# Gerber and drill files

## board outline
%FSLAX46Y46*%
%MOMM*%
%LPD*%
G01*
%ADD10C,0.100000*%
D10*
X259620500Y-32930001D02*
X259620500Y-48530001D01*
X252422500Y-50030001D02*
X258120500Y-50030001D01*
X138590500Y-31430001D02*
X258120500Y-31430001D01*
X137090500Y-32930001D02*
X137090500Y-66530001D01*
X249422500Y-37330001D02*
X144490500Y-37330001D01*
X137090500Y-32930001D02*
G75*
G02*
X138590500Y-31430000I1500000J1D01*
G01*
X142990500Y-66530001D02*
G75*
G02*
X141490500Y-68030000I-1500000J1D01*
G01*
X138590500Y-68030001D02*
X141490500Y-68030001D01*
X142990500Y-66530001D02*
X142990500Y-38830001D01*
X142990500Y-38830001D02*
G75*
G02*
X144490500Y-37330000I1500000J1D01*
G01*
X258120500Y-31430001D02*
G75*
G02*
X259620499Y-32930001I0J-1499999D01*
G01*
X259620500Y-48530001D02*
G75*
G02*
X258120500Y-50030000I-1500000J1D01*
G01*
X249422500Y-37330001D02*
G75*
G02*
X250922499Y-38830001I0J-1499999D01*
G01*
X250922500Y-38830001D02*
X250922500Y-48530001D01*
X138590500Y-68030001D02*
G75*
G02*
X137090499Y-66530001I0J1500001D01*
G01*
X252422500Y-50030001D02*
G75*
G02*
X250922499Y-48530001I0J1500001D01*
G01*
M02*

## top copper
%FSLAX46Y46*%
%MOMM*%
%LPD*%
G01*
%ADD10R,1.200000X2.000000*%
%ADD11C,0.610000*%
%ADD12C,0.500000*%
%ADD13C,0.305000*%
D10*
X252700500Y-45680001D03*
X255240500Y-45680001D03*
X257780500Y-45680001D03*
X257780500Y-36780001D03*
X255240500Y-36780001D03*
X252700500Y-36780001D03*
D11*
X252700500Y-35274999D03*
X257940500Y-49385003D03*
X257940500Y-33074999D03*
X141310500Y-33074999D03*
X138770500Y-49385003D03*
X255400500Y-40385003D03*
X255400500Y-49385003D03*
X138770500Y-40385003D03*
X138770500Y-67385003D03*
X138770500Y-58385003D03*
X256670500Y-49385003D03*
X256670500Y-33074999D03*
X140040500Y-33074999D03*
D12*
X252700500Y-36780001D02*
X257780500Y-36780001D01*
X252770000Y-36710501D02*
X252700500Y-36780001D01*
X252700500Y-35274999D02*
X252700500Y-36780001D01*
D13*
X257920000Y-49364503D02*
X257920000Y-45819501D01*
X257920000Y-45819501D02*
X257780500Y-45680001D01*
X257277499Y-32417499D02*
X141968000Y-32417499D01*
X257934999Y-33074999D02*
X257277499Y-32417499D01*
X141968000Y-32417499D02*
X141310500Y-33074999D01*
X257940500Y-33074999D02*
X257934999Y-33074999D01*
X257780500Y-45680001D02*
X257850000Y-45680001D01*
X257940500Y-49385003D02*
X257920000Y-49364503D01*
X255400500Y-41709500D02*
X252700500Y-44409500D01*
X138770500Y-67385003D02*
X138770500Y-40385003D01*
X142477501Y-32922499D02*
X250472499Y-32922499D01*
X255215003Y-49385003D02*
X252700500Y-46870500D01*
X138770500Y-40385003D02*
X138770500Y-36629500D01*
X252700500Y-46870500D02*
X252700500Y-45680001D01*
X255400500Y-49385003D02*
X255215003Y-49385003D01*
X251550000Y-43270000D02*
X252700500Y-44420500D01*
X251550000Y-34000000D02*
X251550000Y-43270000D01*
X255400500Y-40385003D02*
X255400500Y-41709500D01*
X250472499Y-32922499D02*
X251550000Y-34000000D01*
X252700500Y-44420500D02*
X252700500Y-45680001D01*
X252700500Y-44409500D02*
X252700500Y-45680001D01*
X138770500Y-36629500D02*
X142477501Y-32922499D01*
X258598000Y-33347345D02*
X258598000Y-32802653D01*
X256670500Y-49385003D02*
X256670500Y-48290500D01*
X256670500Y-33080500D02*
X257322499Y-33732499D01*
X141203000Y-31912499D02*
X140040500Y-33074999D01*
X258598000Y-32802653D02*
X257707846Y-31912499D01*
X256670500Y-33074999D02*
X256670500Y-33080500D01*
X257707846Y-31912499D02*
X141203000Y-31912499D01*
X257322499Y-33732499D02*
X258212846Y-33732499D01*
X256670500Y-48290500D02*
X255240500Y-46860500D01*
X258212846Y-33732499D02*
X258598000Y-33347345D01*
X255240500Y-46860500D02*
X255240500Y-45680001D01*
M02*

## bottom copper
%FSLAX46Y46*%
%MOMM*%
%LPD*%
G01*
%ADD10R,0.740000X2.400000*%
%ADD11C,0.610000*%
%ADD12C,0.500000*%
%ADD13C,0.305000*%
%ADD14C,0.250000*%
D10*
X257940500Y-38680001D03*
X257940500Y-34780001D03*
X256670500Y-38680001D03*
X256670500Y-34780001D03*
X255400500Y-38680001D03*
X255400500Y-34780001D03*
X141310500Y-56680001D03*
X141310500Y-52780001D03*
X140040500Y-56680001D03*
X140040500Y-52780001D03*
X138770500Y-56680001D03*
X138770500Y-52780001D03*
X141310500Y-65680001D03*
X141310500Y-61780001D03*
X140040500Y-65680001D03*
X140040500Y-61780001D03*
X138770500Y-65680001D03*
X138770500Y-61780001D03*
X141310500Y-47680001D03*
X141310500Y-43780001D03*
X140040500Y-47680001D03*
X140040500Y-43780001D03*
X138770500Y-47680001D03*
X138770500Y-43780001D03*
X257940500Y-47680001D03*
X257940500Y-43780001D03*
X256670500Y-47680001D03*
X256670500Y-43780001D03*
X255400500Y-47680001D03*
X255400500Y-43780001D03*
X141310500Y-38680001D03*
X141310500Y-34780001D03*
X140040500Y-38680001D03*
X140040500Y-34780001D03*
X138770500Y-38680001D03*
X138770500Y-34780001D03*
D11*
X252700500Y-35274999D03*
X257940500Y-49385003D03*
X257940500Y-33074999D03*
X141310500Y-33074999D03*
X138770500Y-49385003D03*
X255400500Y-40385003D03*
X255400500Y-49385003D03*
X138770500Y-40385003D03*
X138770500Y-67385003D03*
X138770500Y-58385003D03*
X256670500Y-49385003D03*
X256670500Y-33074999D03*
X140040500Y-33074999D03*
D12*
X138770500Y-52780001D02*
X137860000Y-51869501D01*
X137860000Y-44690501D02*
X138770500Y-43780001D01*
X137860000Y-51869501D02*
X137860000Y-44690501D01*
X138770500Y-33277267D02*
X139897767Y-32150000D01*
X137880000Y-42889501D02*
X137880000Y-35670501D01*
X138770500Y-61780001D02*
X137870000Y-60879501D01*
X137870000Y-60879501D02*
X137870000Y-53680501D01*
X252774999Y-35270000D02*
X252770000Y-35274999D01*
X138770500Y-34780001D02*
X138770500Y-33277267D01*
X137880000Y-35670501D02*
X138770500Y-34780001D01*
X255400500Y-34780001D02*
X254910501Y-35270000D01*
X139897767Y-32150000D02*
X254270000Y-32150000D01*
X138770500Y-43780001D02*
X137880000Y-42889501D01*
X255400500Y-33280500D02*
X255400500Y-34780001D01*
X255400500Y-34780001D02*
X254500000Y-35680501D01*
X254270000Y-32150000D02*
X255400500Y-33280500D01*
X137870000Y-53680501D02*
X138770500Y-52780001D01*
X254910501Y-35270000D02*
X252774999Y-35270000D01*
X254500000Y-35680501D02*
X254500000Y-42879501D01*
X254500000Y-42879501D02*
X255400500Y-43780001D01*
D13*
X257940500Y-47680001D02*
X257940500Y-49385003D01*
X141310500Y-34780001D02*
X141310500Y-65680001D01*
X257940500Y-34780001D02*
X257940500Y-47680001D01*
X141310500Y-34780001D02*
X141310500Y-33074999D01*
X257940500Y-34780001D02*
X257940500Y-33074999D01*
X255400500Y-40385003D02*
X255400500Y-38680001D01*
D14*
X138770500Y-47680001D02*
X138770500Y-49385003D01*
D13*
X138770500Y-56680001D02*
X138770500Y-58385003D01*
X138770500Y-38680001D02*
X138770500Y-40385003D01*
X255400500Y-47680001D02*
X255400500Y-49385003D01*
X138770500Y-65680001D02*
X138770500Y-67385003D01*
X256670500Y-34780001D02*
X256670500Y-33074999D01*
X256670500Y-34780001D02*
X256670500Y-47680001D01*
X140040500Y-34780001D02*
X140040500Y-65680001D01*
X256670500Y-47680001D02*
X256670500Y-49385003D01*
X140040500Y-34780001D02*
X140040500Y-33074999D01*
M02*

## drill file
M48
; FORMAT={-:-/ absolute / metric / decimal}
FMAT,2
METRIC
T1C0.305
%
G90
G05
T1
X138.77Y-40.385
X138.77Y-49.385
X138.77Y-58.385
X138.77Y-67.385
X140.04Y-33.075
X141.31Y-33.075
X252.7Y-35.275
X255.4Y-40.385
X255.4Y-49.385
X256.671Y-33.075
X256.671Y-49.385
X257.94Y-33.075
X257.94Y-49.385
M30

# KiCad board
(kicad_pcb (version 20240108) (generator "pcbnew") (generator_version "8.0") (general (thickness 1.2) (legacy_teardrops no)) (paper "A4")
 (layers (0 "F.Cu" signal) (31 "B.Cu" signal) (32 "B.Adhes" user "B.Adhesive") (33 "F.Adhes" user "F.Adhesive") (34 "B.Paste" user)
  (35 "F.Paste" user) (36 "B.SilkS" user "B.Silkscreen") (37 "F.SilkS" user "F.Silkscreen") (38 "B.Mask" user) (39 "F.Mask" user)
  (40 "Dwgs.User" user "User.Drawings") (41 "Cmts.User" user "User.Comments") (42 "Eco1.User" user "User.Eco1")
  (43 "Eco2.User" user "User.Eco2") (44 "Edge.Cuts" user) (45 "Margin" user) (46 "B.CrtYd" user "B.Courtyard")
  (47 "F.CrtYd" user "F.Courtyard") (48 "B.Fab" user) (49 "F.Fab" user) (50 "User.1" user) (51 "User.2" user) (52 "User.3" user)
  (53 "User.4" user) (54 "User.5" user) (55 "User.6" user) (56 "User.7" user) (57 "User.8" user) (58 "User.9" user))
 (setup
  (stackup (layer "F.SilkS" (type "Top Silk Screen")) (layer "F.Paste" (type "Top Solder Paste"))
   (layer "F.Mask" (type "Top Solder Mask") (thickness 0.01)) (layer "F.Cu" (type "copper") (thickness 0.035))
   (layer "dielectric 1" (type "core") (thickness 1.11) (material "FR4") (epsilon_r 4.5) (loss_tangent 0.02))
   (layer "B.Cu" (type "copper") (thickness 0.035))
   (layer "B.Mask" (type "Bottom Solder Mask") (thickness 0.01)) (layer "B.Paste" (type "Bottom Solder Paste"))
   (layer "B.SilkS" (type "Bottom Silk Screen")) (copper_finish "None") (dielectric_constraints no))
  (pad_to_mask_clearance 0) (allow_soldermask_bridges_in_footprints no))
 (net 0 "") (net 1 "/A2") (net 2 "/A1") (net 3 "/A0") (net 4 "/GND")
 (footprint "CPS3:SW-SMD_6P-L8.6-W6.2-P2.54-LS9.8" (layer "F.Cu") (at 255.2405 41.230001)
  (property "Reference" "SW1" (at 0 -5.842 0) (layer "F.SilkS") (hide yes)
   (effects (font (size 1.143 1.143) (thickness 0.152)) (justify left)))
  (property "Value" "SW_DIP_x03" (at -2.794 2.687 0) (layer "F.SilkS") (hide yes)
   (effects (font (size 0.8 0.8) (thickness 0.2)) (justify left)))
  (pad "1" smd rect (at -2.54 4.45) (size 1.2 2) (layers "F.Cu" "F.Paste" "F.Mask") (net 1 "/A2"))
  (pad "2" smd rect (at 0 4.45) (size 1.2 2) (layers "F.Cu" "F.Paste" "F.Mask") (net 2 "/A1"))
  (pad "3" smd rect (at 2.54 4.45) (size 1.2 2) (layers "F.Cu" "F.Paste" "F.Mask") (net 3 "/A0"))
  (pad "4" smd rect (at 2.54 -4.45) (size 1.2 2) (layers "F.Cu" "F.Paste" "F.Mask") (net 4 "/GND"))
  (pad "5" smd rect (at 0 -4.45) (size 1.2 2) (layers "F.Cu" "F.Paste" "F.Mask") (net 4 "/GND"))
  (pad "6" smd rect (at -2.54 -4.45) (size 1.2 2) (layers "F.Cu" "F.Paste" "F.Mask") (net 4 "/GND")))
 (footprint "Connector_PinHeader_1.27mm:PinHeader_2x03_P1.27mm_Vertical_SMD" (layer "B.Cu") (at 256.6705 36.730001 90)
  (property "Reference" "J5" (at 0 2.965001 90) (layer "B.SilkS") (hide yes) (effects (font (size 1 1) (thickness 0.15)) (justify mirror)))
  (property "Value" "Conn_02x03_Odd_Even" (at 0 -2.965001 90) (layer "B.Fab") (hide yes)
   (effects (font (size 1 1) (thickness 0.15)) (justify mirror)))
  (pad "1" smd rect (at -1.95 1.27 90) (size 2.4 0.74) (layers "B.Cu" "B.Paste" "B.Mask") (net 3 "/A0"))
  (pad "2" smd rect (at 1.95 1.27 90) (size 2.4 0.74) (layers "B.Cu" "B.Paste" "B.Mask") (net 3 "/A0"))
  (pad "3" smd rect (at -1.95 0 90) (size 2.4 0.74) (layers "B.Cu" "B.Paste" "B.Mask") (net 2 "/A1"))
  (pad "4" smd rect (at 1.95 0 90) (size 2.4 0.74) (layers "B.Cu" "B.Paste" "B.Mask") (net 2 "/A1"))
  (pad "5" smd rect (at -1.95 -1.27 90) (size 2.4 0.74) (layers "B.Cu" "B.Paste" "B.Mask") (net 1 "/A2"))
  (pad "6" smd rect (at 1.95 -1.27 90) (size 2.4 0.74) (layers "B.Cu" "B.Paste" "B.Mask") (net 4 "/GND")))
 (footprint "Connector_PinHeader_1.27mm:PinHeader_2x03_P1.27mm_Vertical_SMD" (layer "B.Cu") (at 140.0405 54.730001 90)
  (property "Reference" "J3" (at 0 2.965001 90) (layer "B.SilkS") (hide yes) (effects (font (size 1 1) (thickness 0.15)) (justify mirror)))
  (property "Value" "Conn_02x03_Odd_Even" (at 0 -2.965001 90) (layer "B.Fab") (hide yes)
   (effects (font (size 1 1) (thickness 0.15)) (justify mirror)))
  (pad "1" smd rect (at -1.95 1.27 90) (size 2.4 0.74) (layers "B.Cu" "B.Paste" "B.Mask") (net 3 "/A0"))
  (pad "2" smd rect (at 1.95 1.27 90) (size 2.4 0.74) (layers "B.Cu" "B.Paste" "B.Mask") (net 3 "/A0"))
  (pad "3" smd rect (at -1.95 0 90) (size 2.4 0.74) (layers "B.Cu" "B.Paste" "B.Mask") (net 2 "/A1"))
  (pad "4" smd rect (at 1.95 0 90) (size 2.4 0.74) (layers "B.Cu" "B.Paste" "B.Mask") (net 2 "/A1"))
  (pad "5" smd rect (at -1.95 -1.27 90) (size 2.4 0.74) (layers "B.Cu" "B.Paste" "B.Mask") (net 1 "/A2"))
  (pad "6" smd rect (at 1.95 -1.27 90) (size 2.4 0.74) (layers "B.Cu" "B.Paste" "B.Mask") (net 4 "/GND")))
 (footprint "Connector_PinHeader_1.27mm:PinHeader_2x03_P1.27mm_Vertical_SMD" (layer "B.Cu") (at 140.0405 63.730001 90)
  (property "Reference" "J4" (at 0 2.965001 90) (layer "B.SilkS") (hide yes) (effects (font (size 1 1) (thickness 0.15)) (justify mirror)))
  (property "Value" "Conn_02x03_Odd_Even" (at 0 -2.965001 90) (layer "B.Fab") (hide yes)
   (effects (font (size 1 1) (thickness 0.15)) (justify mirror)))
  (pad "1" smd rect (at -1.95 1.27 90) (size 2.4 0.74) (layers "B.Cu" "B.Paste" "B.Mask") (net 3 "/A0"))
  (pad "2" smd rect (at 1.95 1.27 90) (size 2.4 0.74) (layers "B.Cu" "B.Paste" "B.Mask") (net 3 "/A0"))
  (pad "3" smd rect (at -1.95 0 90) (size 2.4 0.74) (layers "B.Cu" "B.Paste" "B.Mask") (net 2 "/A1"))
  (pad "4" smd rect (at 1.95 0 90) (size 2.4 0.74) (layers "B.Cu" "B.Paste" "B.Mask") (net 2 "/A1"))
  (pad "5" smd rect (at -1.95 -1.27 90) (size 2.4 0.74) (layers "B.Cu" "B.Paste" "B.Mask") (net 1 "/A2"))
  (pad "6" smd rect (at 1.95 -1.27 90) (size 2.4 0.74) (layers "B.Cu" "B.Paste" "B.Mask") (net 4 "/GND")))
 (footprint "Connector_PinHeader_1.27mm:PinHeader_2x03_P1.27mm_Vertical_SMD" (layer "B.Cu") (at 140.0405 45.730001 90)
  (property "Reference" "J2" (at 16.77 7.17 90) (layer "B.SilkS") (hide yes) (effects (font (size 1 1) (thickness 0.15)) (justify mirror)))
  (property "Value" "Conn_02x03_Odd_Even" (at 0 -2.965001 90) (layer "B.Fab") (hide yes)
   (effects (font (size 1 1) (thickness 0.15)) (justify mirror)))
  (pad "1" smd rect (at -1.95 1.27 90) (size 2.4 0.74) (layers "B.Cu" "B.Paste" "B.Mask") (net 3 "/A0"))
  (pad "2" smd rect (at 1.95 1.27 90) (size 2.4 0.74) (layers "B.Cu" "B.Paste" "B.Mask") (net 3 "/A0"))
  (pad "3" smd rect (at -1.95 0 90) (size 2.4 0.74) (layers "B.Cu" "B.Paste" "B.Mask") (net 2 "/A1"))
  (pad "4" smd rect (at 1.95 0 90) (size 2.4 0.74) (layers "B.Cu" "B.Paste" "B.Mask") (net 2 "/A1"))
  (pad "5" smd rect (at -1.95 -1.27 90) (size 2.4 0.74) (layers "B.Cu" "B.Paste" "B.Mask") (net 1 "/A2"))
  (pad "6" smd rect (at 1.95 -1.27 90) (size 2.4 0.74) (layers "B.Cu" "B.Paste" "B.Mask") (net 4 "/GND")))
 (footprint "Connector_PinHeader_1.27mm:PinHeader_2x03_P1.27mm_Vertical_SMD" (layer "B.Cu") (at 256.6705 45.730001 90)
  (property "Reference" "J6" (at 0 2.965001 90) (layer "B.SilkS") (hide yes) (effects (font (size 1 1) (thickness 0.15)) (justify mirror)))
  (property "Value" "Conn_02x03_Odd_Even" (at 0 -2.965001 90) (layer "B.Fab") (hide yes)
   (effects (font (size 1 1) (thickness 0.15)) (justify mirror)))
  (pad "1" smd rect (at -1.95 1.27 90) (size 2.4 0.74) (layers "B.Cu" "B.Paste" "B.Mask") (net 3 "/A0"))
  (pad "2" smd rect (at 1.95 1.27 90) (size 2.4 0.74) (layers "B.Cu" "B.Paste" "B.Mask") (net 3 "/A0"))
  (pad "3" smd rect (at -1.95 0 90) (size 2.4 0.74) (layers "B.Cu" "B.Paste" "B.Mask") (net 2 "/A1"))
  (pad "4" smd rect (at 1.95 0 90) (size 2.4 0.74) (layers "B.Cu" "B.Paste" "B.Mask") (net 2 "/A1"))
  (pad "5" smd rect (at -1.95 -1.27 90) (size 2.4 0.74) (layers "B.Cu" "B.Paste" "B.Mask") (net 1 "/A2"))
  (pad "6" smd rect (at 1.95 -1.27 90) (size 2.4 0.74) (layers "B.Cu" "B.Paste" "B.Mask") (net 4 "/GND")))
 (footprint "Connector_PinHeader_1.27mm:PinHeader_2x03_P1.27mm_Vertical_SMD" (layer "B.Cu") (at 140.0405 36.730001 90)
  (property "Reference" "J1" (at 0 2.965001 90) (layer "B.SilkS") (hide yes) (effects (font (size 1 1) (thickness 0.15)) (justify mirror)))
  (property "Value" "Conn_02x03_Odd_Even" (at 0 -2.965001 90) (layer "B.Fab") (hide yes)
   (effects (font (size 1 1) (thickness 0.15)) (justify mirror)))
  (pad "1" smd rect (at -1.95 1.27 90) (size 2.4 0.74) (layers "B.Cu" "B.Paste" "B.Mask") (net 3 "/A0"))
  (pad "2" smd rect (at 1.95 1.27 90) (size 2.4 0.74) (layers "B.Cu" "B.Paste" "B.Mask") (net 3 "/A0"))
  (pad "3" smd rect (at -1.95 0 90) (size 2.4 0.74) (layers "B.Cu" "B.Paste" "B.Mask") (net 2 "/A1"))
  (pad "4" smd rect (at 1.95 0 90) (size 2.4 0.74) (layers "B.Cu" "B.Paste" "B.Mask") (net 2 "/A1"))
  (pad "5" smd rect (at -1.95 -1.27 90) (size 2.4 0.74) (layers "B.Cu" "B.Paste" "B.Mask") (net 1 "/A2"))
  (pad "6" smd rect (at 1.95 -1.27 90) (size 2.4 0.74) (layers "B.Cu" "B.Paste" "B.Mask") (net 4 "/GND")))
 (gr_line (start 259.6205 32.930001) (end 259.6205 48.530001) (stroke (width 0.1) (type default)) (layer "Edge.Cuts"))
 (gr_line (start 252.4225 50.030001) (end 258.1205 50.030001) (stroke (width 0.1) (type default)) (layer "Edge.Cuts"))
 (gr_line (start 138.5905 31.430001) (end 258.1205 31.430001) (stroke (width 0.1) (type default)) (layer "Edge.Cuts"))
 (gr_line (start 137.0905 32.930001) (end 137.0905 66.530001) (stroke (width 0.1) (type default)) (layer "Edge.Cuts"))
 (gr_line (start 249.4225 37.330001) (end 144.4905 37.330001) (stroke (width 0.1) (type default)) (layer "Edge.Cuts"))
 (gr_arc (start 137.0905 32.930001) (mid 137.52984 31.869341) (end 138.5905 31.430001) (stroke (width 0.1) (type default))
  (layer "Edge.Cuts"))
 (gr_arc (start 142.9905 66.530001) (mid 142.55116 67.590661) (end 141.4905 68.030001) (stroke (width 0.1) (type default))
  (layer "Edge.Cuts"))
 (gr_line (start 138.5905 68.030001) (end 141.4905 68.030001) (stroke (width 0.1) (type default)) (layer "Edge.Cuts"))
 (gr_line (start 142.9905 66.530001) (end 142.9905 38.830001) (stroke (width 0.1) (type default)) (layer "Edge.Cuts"))
 (gr_arc (start 142.9905 38.830001) (mid 143.429839 37.76934) (end 144.4905 37.330001) (stroke (width 0.1) (type default))
  (layer "Edge.Cuts"))
 (gr_arc (start 258.1205 31.430001) (mid 259.18116 31.869341) (end 259.6205 32.930001) (stroke (width 0.1) (type default))
  (layer "Edge.Cuts"))
 (gr_arc (start 259.6205 48.530001) (mid 259.18116 49.590661) (end 258.1205 50.030001) (stroke (width 0.1) (type default))
  (layer "Edge.Cuts"))
 (gr_arc (start 249.4225 37.330001) (mid 250.48316 37.769341) (end 250.9225 38.830001) (stroke (width 0.1) (type default))
  (layer "Edge.Cuts"))
 (gr_line (start 250.9225 38.830001) (end 250.9225 48.530001) (stroke (width 0.1) (type default)) (layer "Edge.Cuts"))
 (gr_arc (start 138.5905 68.030001) (mid 137.529839 67.590662) (end 137.0905 66.530001) (stroke (width 0.1) (type default))
  (layer "Edge.Cuts"))
 (gr_arc (start 252.4225 50.030001) (mid 251.361839 49.590662) (end 250.9225 48.530001) (stroke (width 0.1) (type default))
  (layer "Edge.Cuts"))
 (segment (start 252.7005 36.780001) (end 257.7805 36.780001) (width 0.5) (layer "F.Cu") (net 4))
 (segment (start 252.77 36.710501) (end 252.7005 36.780001) (width 0.5) (layer "F.Cu") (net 4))
 (segment (start 252.7005 35.274999) (end 252.7005 36.780001) (width 0.5) (layer "F.Cu") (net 4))
 (via (at 252.7005 35.274999) (size 0.61) (drill 0.305) (layers "F.Cu" "B.Cu") (free yes) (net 4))
 (segment (start 138.7705 52.780001) (end 137.86 51.869501) (width 0.5) (layer "B.Cu") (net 4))
 (segment (start 137.86 44.690501) (end 138.7705 43.780001) (width 0.5) (layer "B.Cu") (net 4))
 (segment (start 137.86 51.869501) (end 137.86 44.690501) (width 0.5) (layer "B.Cu") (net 4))
 (segment (start 138.7705 33.277267) (end 139.897767 32.15) (width 0.5) (layer "B.Cu") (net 4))
 (segment (start 137.88 42.889501) (end 137.88 35.670501) (width 0.5) (layer "B.Cu") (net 4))
 (segment (start 138.7705 61.780001) (end 137.87 60.879501) (width 0.5) (layer "B.Cu") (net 4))
 (segment (start 137.87 60.879501) (end 137.87 53.680501) (width 0.5) (layer "B.Cu") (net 4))
 (segment (start 252.774999 35.27) (end 252.77 35.274999) (width 0.5) (layer "B.Cu") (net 4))
 (segment (start 138.7705 34.780001) (end 138.7705 33.277267) (width 0.5) (layer "B.Cu") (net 4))
 (segment (start 137.88 35.670501) (end 138.7705 34.780001) (width 0.5) (layer "B.Cu") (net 4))
 (segment (start 255.4005 34.780001) (end 254.910501 35.27) (width 0.5) (layer "B.Cu") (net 4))
 (segment (start 139.897767 32.15) (end 254.27 32.15) (width 0.5) (layer "B.Cu") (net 4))
 (segment (start 138.7705 43.780001) (end 137.88 42.889501) (width 0.5) (layer "B.Cu") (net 4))
 (segment (start 255.4005 33.2805) (end 255.4005 34.780001) (width 0.5) (layer "B.Cu") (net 4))
 (segment (start 255.4005 34.780001) (end 254.5 35.680501) (width 0.5) (layer "B.Cu") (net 4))
 (segment (start 254.27 32.15) (end 255.4005 33.2805) (width 0.5) (layer "B.Cu") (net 4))
 (segment (start 137.87 53.680501) (end 138.7705 52.780001) (width 0.5) (layer "B.Cu") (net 4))
 (segment (start 254.910501 35.27) (end 252.774999 35.27) (width 0.5) (layer "B.Cu") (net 4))
 (segment (start 254.5 35.680501) (end 254.5 42.879501) (width 0.5) (layer "B.Cu") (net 4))
 (segment (start 254.5 42.879501) (end 255.4005 43.780001) (width 0.5) (layer "B.Cu") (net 4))
 (segment (start 257.92 49.364503) (end 257.92 45.819501) (width 0.305) (layer "F.Cu") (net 3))
 (segment (start 257.92 45.819501) (end 257.7805 45.680001) (width 0.305) (layer "F.Cu") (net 3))
 (segment (start 257.277499 32.417499) (end 141.968 32.417499) (width 0.305) (layer "F.Cu") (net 3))
 (segment (start 257.934999 33.074999) (end 257.277499 32.417499) (width 0.305) (layer "F.Cu") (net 3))
 (segment (start 141.968 32.417499) (end 141.3105 33.074999) (width 0.305) (layer "F.Cu") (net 3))
 (segment (start 257.9405 33.074999) (end 257.934999 33.074999) (width 0.305) (layer "F.Cu") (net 3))
 (segment (start 257.7805 45.680001) (end 257.85 45.680001) (width 0.305) (layer "F.Cu") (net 3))
 (segment (start 257.9405 49.385003) (end 257.92 49.364503) (width 0.305) (layer "F.Cu") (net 3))
 (via (at 257.9405 49.385003) (size 0.61) (drill 0.305) (layers "F.Cu" "B.Cu") (free yes) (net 3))
 (via (at 257.9405 33.074999) (size 0.61) (drill 0.305) (layers "F.Cu" "B.Cu") (free yes) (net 3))
 (via (at 141.3105 33.074999) (size 0.61) (drill 0.305) (layers "F.Cu" "B.Cu") (free yes) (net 3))
 (segment (start 257.9405 47.680001) (end 257.9405 49.385003) (width 0.305) (layer "B.Cu") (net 3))
 (segment (start 141.3105 34.780001) (end 141.3105 65.680001) (width 0.305) (layer "B.Cu") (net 3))
 (segment (start 257.9405 34.780001) (end 257.9405 47.680001) (width 0.305) (layer "B.Cu") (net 3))
 (segment (start 141.3105 34.780001) (end 141.3105 33.074999) (width 0.305) (layer "B.Cu") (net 3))
 (segment (start 257.9405 34.780001) (end 257.9405 33.074999) (width 0.305) (layer "B.Cu") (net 3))
 (segment (start 255.4005 41.7095) (end 252.7005 44.4095) (width 0.305) (layer "F.Cu") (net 1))
 (segment (start 138.7705 67.385003) (end 138.7705 40.385003) (width 0.305) (layer "F.Cu") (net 1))
 (segment (start 142.477501 32.922499) (end 250.472499 32.922499) (width 0.305) (layer "F.Cu") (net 1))
 (segment (start 255.215003 49.385003) (end 252.7005 46.8705) (width 0.305) (layer "F.Cu") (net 1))
 (segment (start 138.7705 40.385003) (end 138.7705 36.6295) (width 0.305) (layer "F.Cu") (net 1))
 (segment (start 252.7005 46.8705) (end 252.7005 45.680001) (width 0.305) (layer "F.Cu") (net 1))
 (segment (start 255.4005 49.385003) (end 255.215003 49.385003) (width 0.305) (layer "F.Cu") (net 1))
 (segment (start 251.55 43.27) (end 252.7005 44.4205) (width 0.305) (layer "F.Cu") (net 1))
 (segment (start 251.55 34) (end 251.55 43.27) (width 0.305) (layer "F.Cu") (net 1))
 (segment (start 255.4005 40.385003) (end 255.4005 41.7095) (width 0.305) (layer "F.Cu") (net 1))
 (segment (start 250.472499 32.922499) (end 251.55 34) (width 0.305) (layer "F.Cu") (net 1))
 (segment (start 252.7005 44.4205) (end 252.7005 45.680001) (width 0.305) (layer "F.Cu") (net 1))
 (segment (start 252.7005 44.4095) (end 252.7005 45.680001) (width 0.305) (layer "F.Cu") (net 1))
 (segment (start 138.7705 36.6295) (end 142.477501 32.922499) (width 0.305) (layer "F.Cu") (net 1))
 (via (at 138.7705 49.385003) (size 0.61) (drill 0.305) (layers "F.Cu" "B.Cu") (free yes) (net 1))
 (via (at 255.4005 40.385003) (size 0.61) (drill 0.305) (layers "F.Cu" "B.Cu") (free yes) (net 1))
 (via (at 255.4005 49.385003) (size 0.61) (drill 0.305) (layers "F.Cu" "B.Cu") (free yes) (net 1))
 (via (at 138.7705 40.385003) (size 0.61) (drill 0.305) (layers "F.Cu" "B.Cu") (free yes) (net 1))
 (via (at 138.7705 67.385003) (size 0.61) (drill 0.305) (layers "F.Cu" "B.Cu") (free yes) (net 1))
 (via (at 138.7705 58.385003) (size 0.61) (drill 0.305) (layers "F.Cu" "B.Cu") (free yes) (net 1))
 (segment (start 255.4005 40.385003) (end 255.4005 38.680001) (width 0.305) (layer "B.Cu") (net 1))
 (segment (start 138.7705 47.680001) (end 138.7705 49.385003) (width 0.25) (layer "B.Cu") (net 1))
 (segment (start 138.7705 56.680001) (end 138.7705 58.385003) (width 0.305) (layer "B.Cu") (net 1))
 (segment (start 138.7705 38.680001) (end 138.7705 40.385003) (width 0.305) (layer "B.Cu") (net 1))
 (segment (start 255.4005 47.680001) (end 255.4005 49.385003) (width 0.305) (layer "B.Cu") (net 1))
 (segment (start 138.7705 65.680001) (end 138.7705 67.385003) (width 0.305) (layer "B.Cu") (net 1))
 (segment (start 258.598 33.347345) (end 258.598 32.802653) (width 0.305) (layer "F.Cu") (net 2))
 (segment (start 256.6705 49.385003) (end 256.6705 48.2905) (width 0.305) (layer "F.Cu") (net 2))
 (segment (start 256.6705 33.0805) (end 257.322499 33.732499) (width 0.305) (layer "F.Cu") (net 2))
 (segment (start 141.203 31.912499) (end 140.0405 33.074999) (width 0.305) (layer "F.Cu") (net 2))
 (segment (start 258.598 32.802653) (end 257.707846 31.912499) (width 0.305) (layer "F.Cu") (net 2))
 (segment (start 256.6705 33.074999) (end 256.6705 33.0805) (width 0.305) (layer "F.Cu") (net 2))
 (segment (start 257.707846 31.912499) (end 141.203 31.912499) (width 0.305) (layer "F.Cu") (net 2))
 (segment (start 257.322499 33.732499) (end 258.212846 33.732499) (width 0.305) (layer "F.Cu") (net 2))
 (segment (start 256.6705 48.2905) (end 255.2405 46.8605) (width 0.305) (layer "F.Cu") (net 2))
 (segment (start 258.212846 33.732499) (end 258.598 33.347345) (width 0.305) (layer "F.Cu") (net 2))
 (segment (start 255.2405 46.8605) (end 255.2405 45.680001) (width 0.305) (layer "F.Cu") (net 2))
 (via (at 256.6705 49.385003) (size 0.61) (drill 0.305) (layers "F.Cu" "B.Cu") (free yes) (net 2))
 (via (at 256.6705 33.074999) (size 0.61) (drill 0.305) (layers "F.Cu" "B.Cu") (free yes) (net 2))
 (via (at 140.0405 33.074999) (size 0.61) (drill 0.305) (layers "F.Cu" "B.Cu") (free yes) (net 2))
 (segment (start 256.6705 34.780001) (end 256.6705 33.074999) (width 0.305) (layer "B.Cu") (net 2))
 (segment (start 256.6705 34.780001) (end 256.6705 47.680001) (width 0.305) (layer "B.Cu") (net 2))
 (segment (start 140.0405 34.780001) (end 140.0405 65.680001) (width 0.305) (layer "B.Cu") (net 2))
 (segment (start 256.6705 47.680001) (end 256.6705 49.385003) (width 0.305) (layer "B.Cu") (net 2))
 (segment (start 140.0405 34.780001) (end 140.0405 33.074999) (width 0.305) (layer "B.Cu") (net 2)))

